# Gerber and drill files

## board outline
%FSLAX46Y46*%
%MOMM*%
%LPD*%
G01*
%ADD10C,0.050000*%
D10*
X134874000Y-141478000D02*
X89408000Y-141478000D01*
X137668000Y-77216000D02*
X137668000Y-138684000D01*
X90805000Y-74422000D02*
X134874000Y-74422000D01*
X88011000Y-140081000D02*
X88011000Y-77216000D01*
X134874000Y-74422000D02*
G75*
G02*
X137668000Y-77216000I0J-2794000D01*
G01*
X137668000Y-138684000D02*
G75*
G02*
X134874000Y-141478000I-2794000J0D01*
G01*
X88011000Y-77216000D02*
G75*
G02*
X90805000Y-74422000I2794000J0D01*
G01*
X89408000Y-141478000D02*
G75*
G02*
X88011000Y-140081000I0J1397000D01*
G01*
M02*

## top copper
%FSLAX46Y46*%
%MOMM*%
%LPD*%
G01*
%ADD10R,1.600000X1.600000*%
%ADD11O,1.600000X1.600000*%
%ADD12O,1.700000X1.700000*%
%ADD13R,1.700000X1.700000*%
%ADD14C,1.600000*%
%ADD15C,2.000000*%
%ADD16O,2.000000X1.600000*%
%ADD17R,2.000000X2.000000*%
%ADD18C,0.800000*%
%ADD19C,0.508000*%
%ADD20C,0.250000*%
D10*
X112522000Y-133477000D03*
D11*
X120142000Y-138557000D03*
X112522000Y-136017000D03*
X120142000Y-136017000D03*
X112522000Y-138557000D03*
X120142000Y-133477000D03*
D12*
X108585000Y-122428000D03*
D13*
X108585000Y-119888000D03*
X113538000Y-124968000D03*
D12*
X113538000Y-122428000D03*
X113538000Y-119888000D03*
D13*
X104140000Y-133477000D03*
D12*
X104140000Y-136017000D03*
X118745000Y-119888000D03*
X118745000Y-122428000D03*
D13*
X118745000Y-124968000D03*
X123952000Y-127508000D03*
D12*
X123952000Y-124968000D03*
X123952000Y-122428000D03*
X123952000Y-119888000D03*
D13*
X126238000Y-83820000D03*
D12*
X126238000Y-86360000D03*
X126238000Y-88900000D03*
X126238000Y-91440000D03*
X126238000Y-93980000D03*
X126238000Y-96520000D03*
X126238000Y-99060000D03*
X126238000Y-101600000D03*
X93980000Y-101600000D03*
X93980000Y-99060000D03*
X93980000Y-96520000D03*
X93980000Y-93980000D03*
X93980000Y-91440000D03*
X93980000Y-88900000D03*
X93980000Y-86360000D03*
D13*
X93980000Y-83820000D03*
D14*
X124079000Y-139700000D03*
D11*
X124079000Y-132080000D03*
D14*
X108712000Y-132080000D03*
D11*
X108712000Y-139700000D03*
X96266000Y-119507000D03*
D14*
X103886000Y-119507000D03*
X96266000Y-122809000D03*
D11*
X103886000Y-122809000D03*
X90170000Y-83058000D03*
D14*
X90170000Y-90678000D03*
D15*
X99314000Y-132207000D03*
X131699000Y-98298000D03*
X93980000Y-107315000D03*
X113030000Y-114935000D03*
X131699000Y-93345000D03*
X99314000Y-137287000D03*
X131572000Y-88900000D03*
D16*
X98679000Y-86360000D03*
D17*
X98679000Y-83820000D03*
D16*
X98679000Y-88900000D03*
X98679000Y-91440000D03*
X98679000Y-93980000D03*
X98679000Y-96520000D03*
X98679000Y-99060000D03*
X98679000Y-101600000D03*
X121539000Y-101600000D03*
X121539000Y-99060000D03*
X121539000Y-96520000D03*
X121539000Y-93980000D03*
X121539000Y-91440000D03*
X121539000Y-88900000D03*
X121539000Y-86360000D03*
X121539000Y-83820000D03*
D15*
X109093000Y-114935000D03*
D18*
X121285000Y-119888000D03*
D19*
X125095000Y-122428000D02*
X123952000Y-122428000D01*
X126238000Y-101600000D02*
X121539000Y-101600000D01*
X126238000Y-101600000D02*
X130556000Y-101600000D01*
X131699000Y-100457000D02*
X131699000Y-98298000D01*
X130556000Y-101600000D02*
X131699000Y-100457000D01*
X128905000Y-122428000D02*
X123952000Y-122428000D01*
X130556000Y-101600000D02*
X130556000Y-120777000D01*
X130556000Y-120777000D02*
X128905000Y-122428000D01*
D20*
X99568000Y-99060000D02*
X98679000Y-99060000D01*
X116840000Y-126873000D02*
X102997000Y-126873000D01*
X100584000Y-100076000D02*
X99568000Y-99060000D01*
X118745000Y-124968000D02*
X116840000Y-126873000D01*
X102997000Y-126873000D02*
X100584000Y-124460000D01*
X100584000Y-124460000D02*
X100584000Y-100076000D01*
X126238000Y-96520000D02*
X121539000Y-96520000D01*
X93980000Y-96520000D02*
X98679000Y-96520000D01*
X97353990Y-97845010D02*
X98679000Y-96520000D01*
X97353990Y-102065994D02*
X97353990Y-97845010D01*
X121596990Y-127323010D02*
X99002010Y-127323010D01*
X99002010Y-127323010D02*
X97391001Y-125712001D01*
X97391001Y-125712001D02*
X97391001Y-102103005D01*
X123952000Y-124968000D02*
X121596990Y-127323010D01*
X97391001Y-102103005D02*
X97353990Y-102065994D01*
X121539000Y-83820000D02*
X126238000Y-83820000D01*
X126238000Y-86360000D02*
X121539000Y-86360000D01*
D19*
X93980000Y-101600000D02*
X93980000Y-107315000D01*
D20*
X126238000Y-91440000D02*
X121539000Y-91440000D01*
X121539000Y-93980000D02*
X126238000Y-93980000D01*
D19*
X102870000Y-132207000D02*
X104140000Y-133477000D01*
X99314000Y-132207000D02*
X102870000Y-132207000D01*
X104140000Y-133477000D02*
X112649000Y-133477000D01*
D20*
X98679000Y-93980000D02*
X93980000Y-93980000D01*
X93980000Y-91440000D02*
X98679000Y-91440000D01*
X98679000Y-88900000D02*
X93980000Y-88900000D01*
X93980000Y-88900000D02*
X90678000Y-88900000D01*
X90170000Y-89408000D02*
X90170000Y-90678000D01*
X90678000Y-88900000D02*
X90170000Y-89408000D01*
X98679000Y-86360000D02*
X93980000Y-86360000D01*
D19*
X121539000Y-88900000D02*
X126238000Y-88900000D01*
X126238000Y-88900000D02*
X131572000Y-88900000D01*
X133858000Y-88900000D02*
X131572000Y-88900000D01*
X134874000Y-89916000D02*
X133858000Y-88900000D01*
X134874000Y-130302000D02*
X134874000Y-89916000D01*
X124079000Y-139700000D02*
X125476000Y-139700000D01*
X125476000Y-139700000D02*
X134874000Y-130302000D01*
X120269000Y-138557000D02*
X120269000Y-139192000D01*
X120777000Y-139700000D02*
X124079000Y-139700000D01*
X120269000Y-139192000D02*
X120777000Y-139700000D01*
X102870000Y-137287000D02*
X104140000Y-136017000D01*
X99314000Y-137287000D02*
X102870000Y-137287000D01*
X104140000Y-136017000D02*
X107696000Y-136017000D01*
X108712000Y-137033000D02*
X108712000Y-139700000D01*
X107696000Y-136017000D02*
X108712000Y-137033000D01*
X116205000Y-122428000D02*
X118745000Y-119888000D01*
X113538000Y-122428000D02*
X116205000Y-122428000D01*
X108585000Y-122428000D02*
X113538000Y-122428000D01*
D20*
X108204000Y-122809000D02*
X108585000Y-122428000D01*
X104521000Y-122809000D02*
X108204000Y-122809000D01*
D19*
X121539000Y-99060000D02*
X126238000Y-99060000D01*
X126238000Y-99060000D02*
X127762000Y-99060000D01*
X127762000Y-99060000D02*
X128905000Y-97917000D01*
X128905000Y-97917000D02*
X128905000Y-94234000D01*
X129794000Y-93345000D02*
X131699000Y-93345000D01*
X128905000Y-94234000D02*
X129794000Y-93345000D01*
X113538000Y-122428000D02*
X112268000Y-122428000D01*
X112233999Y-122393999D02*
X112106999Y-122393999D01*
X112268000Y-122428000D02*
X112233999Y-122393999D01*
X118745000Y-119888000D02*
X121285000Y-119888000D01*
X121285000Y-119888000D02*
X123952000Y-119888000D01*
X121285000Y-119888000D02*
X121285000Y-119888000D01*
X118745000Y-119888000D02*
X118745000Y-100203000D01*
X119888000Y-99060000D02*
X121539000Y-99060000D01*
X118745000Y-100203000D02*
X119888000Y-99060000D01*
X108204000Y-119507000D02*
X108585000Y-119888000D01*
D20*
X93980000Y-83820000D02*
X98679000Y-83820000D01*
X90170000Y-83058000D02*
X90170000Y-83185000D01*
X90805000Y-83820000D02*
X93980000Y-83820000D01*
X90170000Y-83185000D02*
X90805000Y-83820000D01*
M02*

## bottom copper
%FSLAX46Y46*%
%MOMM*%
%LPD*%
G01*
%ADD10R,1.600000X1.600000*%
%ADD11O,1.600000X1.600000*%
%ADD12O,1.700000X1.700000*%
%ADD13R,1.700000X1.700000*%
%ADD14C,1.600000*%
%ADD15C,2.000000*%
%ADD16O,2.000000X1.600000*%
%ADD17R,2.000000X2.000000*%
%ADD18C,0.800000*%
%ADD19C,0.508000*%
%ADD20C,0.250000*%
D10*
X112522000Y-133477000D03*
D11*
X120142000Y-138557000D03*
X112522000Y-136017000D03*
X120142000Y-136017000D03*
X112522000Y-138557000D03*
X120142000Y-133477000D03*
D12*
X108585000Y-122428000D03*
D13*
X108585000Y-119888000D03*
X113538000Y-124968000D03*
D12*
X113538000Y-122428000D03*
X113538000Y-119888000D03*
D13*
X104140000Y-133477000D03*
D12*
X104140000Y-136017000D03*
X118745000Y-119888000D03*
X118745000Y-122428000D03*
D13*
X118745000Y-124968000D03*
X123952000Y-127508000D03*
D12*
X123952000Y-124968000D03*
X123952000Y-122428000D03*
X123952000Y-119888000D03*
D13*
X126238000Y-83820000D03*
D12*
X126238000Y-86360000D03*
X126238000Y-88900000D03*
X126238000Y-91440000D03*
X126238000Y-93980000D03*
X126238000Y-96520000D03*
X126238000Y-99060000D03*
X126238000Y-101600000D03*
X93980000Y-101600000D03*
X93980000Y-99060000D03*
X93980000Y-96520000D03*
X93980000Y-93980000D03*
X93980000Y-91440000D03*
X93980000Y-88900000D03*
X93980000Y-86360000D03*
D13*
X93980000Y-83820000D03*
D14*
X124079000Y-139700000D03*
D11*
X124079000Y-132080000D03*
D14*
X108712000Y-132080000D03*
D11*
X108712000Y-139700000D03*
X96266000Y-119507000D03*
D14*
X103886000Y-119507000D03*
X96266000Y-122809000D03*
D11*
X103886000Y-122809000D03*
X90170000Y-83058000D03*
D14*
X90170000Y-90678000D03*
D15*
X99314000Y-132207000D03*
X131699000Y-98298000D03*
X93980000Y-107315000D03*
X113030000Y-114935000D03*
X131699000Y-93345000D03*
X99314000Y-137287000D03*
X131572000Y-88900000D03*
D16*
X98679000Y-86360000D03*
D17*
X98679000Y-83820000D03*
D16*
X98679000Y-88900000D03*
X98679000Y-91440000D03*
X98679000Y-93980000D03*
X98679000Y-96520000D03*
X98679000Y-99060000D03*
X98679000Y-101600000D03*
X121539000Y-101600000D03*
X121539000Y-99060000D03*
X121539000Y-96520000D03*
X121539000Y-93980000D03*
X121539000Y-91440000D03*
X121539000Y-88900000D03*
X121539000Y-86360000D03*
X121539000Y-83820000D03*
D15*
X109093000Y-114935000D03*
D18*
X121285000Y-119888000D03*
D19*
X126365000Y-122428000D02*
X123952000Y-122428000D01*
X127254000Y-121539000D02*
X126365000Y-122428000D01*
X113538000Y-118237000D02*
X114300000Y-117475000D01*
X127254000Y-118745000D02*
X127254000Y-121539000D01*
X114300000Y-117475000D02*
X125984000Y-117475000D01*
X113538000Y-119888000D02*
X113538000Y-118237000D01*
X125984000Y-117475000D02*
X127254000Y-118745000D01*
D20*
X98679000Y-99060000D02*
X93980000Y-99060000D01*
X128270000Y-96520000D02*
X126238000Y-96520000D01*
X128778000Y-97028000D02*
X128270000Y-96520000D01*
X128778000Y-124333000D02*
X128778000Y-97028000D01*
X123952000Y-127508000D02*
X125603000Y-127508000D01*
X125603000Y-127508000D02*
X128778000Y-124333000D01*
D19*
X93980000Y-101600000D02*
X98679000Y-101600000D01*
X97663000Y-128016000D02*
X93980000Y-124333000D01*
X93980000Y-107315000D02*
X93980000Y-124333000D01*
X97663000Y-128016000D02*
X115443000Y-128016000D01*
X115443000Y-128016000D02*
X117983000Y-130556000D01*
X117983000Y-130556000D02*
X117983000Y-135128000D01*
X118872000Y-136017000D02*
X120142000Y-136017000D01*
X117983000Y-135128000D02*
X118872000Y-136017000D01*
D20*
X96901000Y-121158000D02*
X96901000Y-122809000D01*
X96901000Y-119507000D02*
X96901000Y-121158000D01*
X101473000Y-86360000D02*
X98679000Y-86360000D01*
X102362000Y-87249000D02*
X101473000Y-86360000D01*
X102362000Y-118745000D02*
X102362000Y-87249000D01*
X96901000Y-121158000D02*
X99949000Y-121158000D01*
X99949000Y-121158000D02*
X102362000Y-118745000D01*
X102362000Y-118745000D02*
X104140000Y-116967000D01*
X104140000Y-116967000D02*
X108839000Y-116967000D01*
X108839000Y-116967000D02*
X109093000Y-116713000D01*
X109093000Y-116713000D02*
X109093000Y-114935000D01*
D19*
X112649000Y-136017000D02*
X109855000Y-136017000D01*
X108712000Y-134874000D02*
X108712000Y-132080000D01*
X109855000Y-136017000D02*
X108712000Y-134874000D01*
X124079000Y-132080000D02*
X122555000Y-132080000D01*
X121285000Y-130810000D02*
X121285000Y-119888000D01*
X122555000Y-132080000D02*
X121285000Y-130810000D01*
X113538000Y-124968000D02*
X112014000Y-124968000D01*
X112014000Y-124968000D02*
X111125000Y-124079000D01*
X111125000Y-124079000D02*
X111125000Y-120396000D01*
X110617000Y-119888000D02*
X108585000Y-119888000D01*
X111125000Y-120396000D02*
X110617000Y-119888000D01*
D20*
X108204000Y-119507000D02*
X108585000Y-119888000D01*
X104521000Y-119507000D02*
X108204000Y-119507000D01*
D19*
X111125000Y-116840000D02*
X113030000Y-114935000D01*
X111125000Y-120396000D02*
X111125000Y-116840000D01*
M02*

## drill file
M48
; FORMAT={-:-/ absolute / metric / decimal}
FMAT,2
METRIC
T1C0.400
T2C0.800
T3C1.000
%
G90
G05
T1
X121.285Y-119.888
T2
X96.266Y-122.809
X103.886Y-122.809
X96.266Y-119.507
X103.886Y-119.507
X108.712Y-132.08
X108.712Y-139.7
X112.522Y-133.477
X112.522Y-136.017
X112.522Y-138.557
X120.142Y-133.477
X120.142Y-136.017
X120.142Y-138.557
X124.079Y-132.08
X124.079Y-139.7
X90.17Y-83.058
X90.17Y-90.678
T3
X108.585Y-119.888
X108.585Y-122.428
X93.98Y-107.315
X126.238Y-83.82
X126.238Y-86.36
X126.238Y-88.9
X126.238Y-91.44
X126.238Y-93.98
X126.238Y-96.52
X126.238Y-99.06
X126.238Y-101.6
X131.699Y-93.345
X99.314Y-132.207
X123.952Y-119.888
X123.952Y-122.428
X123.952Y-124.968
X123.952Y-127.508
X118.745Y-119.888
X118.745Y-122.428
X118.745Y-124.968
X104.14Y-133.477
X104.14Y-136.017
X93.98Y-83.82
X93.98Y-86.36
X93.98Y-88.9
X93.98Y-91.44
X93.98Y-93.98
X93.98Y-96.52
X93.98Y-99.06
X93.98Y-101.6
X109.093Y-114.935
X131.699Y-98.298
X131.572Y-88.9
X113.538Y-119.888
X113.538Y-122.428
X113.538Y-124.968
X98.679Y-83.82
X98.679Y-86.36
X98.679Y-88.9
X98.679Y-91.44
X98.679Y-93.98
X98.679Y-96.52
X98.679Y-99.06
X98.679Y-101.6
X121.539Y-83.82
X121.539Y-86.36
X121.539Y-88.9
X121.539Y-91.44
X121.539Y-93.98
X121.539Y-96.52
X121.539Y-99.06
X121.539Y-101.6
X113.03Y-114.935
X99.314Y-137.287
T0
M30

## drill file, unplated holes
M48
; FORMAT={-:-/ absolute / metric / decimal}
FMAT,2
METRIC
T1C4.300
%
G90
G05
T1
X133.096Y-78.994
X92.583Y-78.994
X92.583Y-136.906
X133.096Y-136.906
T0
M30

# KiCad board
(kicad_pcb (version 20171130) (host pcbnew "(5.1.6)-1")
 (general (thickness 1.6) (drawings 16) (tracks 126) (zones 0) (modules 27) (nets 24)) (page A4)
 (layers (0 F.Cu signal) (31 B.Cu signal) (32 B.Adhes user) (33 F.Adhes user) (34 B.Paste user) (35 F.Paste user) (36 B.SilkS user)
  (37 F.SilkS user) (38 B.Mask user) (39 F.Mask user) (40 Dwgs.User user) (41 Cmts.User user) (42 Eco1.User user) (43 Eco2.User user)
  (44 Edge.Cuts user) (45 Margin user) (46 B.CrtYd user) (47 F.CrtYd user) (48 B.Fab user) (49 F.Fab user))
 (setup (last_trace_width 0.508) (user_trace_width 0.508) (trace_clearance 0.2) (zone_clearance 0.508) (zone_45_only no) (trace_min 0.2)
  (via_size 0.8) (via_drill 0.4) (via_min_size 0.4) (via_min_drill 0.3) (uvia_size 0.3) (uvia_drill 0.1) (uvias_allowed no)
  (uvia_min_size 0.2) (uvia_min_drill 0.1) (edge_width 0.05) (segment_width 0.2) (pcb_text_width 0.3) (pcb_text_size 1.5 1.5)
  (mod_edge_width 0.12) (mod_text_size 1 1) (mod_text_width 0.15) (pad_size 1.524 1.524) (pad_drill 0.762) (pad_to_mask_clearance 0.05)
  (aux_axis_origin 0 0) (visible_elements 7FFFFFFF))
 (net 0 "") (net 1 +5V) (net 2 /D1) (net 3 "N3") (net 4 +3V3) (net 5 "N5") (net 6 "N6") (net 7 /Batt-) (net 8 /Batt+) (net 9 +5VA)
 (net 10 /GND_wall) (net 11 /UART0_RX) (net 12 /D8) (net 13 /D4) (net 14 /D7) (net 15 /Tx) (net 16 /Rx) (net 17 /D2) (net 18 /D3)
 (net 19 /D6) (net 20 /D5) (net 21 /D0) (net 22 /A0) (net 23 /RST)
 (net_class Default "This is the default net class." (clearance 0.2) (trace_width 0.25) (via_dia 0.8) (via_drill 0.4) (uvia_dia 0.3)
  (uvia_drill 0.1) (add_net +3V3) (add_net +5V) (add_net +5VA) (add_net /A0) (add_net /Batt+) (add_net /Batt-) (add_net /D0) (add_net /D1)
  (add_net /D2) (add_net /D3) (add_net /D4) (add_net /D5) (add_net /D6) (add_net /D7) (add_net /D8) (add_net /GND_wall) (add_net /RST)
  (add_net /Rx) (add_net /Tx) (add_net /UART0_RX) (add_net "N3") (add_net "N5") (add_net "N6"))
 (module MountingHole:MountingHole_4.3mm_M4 (layer F.Cu) (at 92.583 136.906)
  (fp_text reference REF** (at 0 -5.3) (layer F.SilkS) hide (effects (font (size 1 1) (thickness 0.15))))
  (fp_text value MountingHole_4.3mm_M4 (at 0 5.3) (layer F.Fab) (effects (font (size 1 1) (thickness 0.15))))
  (pad 1 np_thru_hole circle (at 0 0) (size 4.3 4.3) (drill 4.3) (layers *.Cu *.Mask)))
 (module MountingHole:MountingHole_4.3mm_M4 (layer F.Cu) (at 133.096 136.906)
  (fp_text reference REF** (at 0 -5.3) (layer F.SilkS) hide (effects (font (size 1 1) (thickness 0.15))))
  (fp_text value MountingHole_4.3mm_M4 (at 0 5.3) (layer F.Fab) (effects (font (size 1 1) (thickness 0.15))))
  (pad 1 np_thru_hole circle (at 0 0) (size 4.3 4.3) (drill 4.3) (layers *.Cu *.Mask)))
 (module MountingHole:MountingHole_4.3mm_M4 (layer F.Cu) (at 92.583 78.994)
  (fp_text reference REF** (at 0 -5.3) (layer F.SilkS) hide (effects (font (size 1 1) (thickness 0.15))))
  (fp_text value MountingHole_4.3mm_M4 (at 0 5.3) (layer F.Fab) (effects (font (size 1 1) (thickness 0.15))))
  (pad 1 np_thru_hole circle (at 0 0) (size 4.3 4.3) (drill 4.3) (layers *.Cu *.Mask)))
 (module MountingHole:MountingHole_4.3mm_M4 (layer F.Cu) (at 133.096 78.994)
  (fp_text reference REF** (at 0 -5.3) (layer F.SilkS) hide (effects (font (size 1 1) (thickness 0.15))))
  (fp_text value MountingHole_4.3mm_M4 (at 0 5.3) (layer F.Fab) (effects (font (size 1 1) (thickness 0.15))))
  (pad 1 np_thru_hole circle (at 0 0) (size 4.3 4.3) (drill 4.3) (layers *.Cu *.Mask)))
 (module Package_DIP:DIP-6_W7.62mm (layer F.Cu) (at 112.522 133.477)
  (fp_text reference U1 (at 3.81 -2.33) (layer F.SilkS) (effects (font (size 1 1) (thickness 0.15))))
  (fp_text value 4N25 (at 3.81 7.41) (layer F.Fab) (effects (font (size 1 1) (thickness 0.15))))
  (pad 1 thru_hole rect (at 0 0) (size 1.6 1.6) (drill 0.8) (layers *.Cu *.Mask) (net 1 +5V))
  (pad 4 thru_hole oval (at 7.62 5.08) (size 1.6 1.6) (drill 0.8) (layers *.Cu *.Mask) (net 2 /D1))
  (pad 2 thru_hole oval (at 0 2.54) (size 1.6 1.6) (drill 0.8) (layers *.Cu *.Mask) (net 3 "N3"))
  (pad 5 thru_hole oval (at 7.62 2.54) (size 1.6 1.6) (drill 0.8) (layers *.Cu *.Mask) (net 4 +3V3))
  (pad 3 thru_hole oval (at 0 5.08) (size 1.6 1.6) (drill 0.8) (layers *.Cu *.Mask) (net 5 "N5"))
  (pad 6 thru_hole oval (at 7.62 0) (size 1.6 1.6) (drill 0.8) (layers *.Cu *.Mask) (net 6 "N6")))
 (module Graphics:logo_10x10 (layer B.Cu) (at 110.109 94.488 180)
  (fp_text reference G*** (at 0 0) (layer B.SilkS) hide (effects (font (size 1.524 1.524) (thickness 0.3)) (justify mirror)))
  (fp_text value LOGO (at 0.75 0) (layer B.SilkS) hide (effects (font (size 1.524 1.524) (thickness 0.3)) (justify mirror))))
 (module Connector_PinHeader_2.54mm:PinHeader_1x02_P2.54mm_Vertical (layer F.Cu) (at 108.585 119.888)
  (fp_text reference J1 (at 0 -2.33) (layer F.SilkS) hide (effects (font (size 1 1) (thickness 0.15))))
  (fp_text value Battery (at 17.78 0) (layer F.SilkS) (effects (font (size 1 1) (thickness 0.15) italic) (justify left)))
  (pad 2 thru_hole oval (at 0 2.54) (size 1.7 1.7) (drill 1) (layers *.Cu *.Mask) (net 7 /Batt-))
  (pad 1 thru_hole rect (at 0 0) (size 1.7 1.7) (drill 1) (layers *.Cu *.Mask) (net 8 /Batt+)))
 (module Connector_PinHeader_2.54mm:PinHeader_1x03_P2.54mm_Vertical (layer F.Cu) (at 113.538 124.968 180)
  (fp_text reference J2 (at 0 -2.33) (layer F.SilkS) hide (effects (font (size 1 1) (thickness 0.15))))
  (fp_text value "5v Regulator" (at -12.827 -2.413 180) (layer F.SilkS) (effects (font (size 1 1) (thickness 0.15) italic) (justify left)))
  (pad 1 thru_hole rect (at 0 0 180) (size 1.7 1.7) (drill 1) (layers *.Cu *.Mask) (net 8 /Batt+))
  (pad 2 thru_hole oval (at 0 2.54 180) (size 1.7 1.7) (drill 1) (layers *.Cu *.Mask) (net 7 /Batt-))
  (pad 3 thru_hole oval (at 0 5.08 180) (size 1.7 1.7) (drill 1) (layers *.Cu *.Mask) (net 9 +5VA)))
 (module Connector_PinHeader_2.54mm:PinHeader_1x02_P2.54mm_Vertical (layer F.Cu) (at 104.14 133.477)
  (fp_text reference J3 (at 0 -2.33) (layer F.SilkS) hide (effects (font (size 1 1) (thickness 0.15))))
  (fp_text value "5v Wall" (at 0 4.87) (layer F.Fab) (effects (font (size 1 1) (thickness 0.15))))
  (pad 1 thru_hole rect (at 0 0) (size 1.7 1.7) (drill 1) (layers *.Cu *.Mask) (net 1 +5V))
  (pad 2 thru_hole oval (at 0 2.54) (size 1.7 1.7) (drill 1) (layers *.Cu *.Mask) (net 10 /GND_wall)))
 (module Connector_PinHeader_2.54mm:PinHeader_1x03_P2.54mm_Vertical (layer F.Cu) (at 118.745 124.968 180)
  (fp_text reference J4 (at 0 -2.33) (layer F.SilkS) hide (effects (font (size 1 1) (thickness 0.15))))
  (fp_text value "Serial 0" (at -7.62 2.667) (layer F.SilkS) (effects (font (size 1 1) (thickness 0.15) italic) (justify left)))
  (pad 3 thru_hole oval (at 0 5.08 180) (size 1.7 1.7) (drill 1) (layers *.Cu *.Mask) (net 7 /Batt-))
  (pad 2 thru_hole oval (at 0 2.54 180) (size 1.7 1.7) (drill 1) (layers *.Cu *.Mask) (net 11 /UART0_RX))
  (pad 1 thru_hole rect (at 0 0 180) (size 1.7 1.7) (drill 1) (layers *.Cu *.Mask) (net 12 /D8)))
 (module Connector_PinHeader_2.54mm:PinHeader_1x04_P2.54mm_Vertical (layer F.Cu) (at 123.952 127.508 180)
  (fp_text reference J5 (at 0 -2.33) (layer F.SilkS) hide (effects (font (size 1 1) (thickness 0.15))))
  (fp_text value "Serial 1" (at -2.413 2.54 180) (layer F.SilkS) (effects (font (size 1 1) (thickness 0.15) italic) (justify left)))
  (pad 1 thru_hole rect (at 0 0 180) (size 1.7 1.7) (drill 1) (layers *.Cu *.Mask) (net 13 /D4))
  (pad 2 thru_hole oval (at 0 2.54 180) (size 1.7 1.7) (drill 1) (layers *.Cu *.Mask) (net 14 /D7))
  (pad 3 thru_hole oval (at 0 5.08 180) (size 1.7 1.7) (drill 1) (layers *.Cu *.Mask) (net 9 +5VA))
  (pad 4 thru_hole oval (at 0 7.62 180) (size 1.7 1.7) (drill 1) (layers *.Cu *.Mask) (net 7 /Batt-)))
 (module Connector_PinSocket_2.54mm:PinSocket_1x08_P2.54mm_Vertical (layer F.Cu) (at 126.238 83.82)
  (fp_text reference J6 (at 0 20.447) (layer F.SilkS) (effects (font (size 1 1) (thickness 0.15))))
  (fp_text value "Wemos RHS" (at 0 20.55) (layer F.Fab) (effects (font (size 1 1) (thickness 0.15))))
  (pad 1 thru_hole rect (at 0 0) (size 1.7 1.7) (drill 1) (layers *.Cu *.Mask) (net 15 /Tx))
  (pad 2 thru_hole oval (at 0 2.54) (size 1.7 1.7) (drill 1) (layers *.Cu *.Mask) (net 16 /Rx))
  (pad 3 thru_hole oval (at 0 5.08) (size 1.7 1.7) (drill 1) (layers *.Cu *.Mask) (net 2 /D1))
  (pad 4 thru_hole oval (at 0 7.62) (size 1.7 1.7) (drill 1) (layers *.Cu *.Mask) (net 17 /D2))
  (pad 5 thru_hole oval (at 0 10.16) (size 1.7 1.7) (drill 1) (layers *.Cu *.Mask) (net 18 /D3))
  (pad 6 thru_hole oval (at 0 12.7) (size 1.7 1.7) (drill 1) (layers *.Cu *.Mask) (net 13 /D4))
  (pad 7 thru_hole oval (at 0 15.24) (size 1.7 1.7) (drill 1) (layers *.Cu *.Mask) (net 7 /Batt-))
  (pad 8 thru_hole oval (at 0 17.78) (size 1.7 1.7) (drill 1) (layers *.Cu *.Mask) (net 9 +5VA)))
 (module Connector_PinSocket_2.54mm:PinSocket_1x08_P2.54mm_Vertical (layer F.Cu) (at 93.98 83.82)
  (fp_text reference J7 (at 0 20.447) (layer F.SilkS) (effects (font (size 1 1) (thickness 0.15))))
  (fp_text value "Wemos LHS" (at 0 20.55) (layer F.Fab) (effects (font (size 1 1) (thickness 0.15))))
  (pad 8 thru_hole oval (at 0 17.78) (size 1.7 1.7) (drill 1) (layers *.Cu *.Mask) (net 4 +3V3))
  (pad 7 thru_hole oval (at 0 15.24) (size 1.7 1.7) (drill 1) (layers *.Cu *.Mask) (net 12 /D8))
  (pad 6 thru_hole oval (at 0 12.7) (size 1.7 1.7) (drill 1) (layers *.Cu *.Mask) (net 14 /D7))
  (pad 5 thru_hole oval (at 0 10.16) (size 1.7 1.7) (drill 1) (layers *.Cu *.Mask) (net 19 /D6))
  (pad 4 thru_hole oval (at 0 7.62) (size 1.7 1.7) (drill 1) (layers *.Cu *.Mask) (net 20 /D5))
  (pad 3 thru_hole oval (at 0 5.08) (size 1.7 1.7) (drill 1) (layers *.Cu *.Mask) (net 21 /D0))
  (pad 2 thru_hole oval (at 0 2.54) (size 1.7 1.7) (drill 1) (layers *.Cu *.Mask) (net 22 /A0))
  (pad 1 thru_hole rect (at 0 0) (size 1.7 1.7) (drill 1) (layers *.Cu *.Mask) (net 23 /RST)))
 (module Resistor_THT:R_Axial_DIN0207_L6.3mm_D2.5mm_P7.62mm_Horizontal (layer F.Cu) (at 124.079 139.7 90)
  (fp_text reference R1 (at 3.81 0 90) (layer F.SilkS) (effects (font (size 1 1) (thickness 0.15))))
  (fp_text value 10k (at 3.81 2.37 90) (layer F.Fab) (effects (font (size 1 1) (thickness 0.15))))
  (pad 1 thru_hole circle (at 0 0 90) (size 1.6 1.6) (drill 0.8) (layers *.Cu *.Mask) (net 2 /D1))
  (pad 2 thru_hole oval (at 7.62 0 90) (size 1.6 1.6) (drill 0.8) (layers *.Cu *.Mask) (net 7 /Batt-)))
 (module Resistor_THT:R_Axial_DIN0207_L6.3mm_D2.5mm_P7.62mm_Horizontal (layer F.Cu) (at 108.712 132.08 270)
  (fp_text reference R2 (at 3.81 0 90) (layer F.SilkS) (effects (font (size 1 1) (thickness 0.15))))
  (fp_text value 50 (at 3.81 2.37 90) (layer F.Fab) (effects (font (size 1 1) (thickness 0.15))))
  (pad 1 thru_hole circle (at 0 0 270) (size 1.6 1.6) (drill 0.8) (layers *.Cu *.Mask) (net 3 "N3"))
  (pad 2 thru_hole oval (at 7.62 0 270) (size 1.6 1.6) (drill 0.8) (layers *.Cu *.Mask) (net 10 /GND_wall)))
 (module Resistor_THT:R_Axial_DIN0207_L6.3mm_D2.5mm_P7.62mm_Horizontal (layer F.Cu) (at 103.886 119.507 180)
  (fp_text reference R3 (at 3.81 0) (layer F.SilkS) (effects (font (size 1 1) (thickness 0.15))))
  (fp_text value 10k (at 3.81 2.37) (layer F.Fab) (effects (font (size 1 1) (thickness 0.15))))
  (pad 2 thru_hole oval (at 7.62 0 180) (size 1.6 1.6) (drill 0.8) (layers *.Cu *.Mask) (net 22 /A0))
  (pad 1 thru_hole circle (at 0 0 180) (size 1.6 1.6) (drill 0.8) (layers *.Cu *.Mask) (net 8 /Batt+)))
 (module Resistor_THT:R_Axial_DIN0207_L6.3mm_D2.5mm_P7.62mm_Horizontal (layer F.Cu) (at 96.266 122.809)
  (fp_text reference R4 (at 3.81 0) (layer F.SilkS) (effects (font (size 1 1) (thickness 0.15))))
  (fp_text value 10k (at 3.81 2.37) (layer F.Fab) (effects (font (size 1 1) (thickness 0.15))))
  (pad 1 thru_hole circle (at 0 0) (size 1.6 1.6) (drill 0.8) (layers *.Cu *.Mask) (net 22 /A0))
  (pad 2 thru_hole oval (at 7.62 0) (size 1.6 1.6) (drill 0.8) (layers *.Cu *.Mask) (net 7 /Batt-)))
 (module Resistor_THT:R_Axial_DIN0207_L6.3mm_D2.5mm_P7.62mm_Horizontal (layer F.Cu) (at 90.17 90.678 90)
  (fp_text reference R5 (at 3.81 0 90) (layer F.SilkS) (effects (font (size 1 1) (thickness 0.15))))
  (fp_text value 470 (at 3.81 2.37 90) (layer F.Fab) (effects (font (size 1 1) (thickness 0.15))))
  (pad 2 thru_hole oval (at 7.62 0 90) (size 1.6 1.6) (drill 0.8) (layers *.Cu *.Mask) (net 23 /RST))
  (pad 1 thru_hole circle (at 0 0 90) (size 1.6 1.6) (drill 0.8) (layers *.Cu *.Mask) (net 21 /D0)))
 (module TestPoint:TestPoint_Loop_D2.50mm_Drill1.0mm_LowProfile (layer F.Cu) (at 99.314 132.207)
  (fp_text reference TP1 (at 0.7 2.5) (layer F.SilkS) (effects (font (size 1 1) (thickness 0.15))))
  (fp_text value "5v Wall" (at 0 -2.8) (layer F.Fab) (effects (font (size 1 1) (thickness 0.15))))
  (pad 1 thru_hole circle (at 0 0) (size 2 2) (drill 1) (layers *.Cu *.Mask) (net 1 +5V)))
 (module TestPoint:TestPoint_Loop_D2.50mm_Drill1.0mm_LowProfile (layer F.Cu) (at 131.699 98.298)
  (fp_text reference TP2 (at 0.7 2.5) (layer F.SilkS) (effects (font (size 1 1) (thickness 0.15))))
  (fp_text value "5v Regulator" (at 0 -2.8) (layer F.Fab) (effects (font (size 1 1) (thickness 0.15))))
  (pad 1 thru_hole circle (at 0 0) (size 2 2) (drill 1) (layers *.Cu *.Mask) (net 9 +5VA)))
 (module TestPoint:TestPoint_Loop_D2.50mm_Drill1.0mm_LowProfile (layer F.Cu) (at 93.98 107.315)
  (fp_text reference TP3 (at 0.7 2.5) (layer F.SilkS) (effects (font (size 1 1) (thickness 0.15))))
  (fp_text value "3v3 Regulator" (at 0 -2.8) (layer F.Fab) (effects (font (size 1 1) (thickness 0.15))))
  (pad 1 thru_hole circle (at 0 0) (size 2 2) (drill 1) (layers *.Cu *.Mask) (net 4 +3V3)))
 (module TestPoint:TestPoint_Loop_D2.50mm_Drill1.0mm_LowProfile (layer F.Cu) (at 113.03 114.935)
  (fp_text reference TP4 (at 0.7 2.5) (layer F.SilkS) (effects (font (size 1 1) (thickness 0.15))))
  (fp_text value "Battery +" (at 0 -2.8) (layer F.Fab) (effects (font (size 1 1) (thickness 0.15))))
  (pad 1 thru_hole circle (at 0 0) (size 2 2) (drill 1) (layers *.Cu *.Mask) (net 8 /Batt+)))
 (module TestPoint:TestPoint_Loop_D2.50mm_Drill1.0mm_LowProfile (layer F.Cu) (at 131.699 93.345)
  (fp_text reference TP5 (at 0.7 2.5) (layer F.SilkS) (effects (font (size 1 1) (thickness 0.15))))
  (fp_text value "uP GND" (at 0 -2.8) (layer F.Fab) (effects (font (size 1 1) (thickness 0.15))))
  (pad 1 thru_hole circle (at 0 0) (size 2 2) (drill 1) (layers *.Cu *.Mask) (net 7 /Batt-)))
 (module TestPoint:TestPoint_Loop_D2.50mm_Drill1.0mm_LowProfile (layer F.Cu) (at 99.314 137.287)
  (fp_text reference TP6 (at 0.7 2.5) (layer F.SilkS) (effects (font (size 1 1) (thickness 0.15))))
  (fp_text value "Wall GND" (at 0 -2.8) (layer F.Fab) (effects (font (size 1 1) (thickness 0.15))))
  (pad 1 thru_hole circle (at 0 0) (size 2 2) (drill 1) (layers *.Cu *.Mask) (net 10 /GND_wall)))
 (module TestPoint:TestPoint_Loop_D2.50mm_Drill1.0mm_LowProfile (layer F.Cu) (at 131.572 88.9)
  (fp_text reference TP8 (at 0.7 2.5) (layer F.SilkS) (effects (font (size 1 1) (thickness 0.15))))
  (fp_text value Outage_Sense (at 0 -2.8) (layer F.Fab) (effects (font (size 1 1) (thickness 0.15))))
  (pad 1 thru_hole circle (at 0 0) (size 2 2) (drill 1) (layers *.Cu *.Mask) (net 2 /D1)))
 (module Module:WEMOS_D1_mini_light (layer F.Cu) (at 98.679 83.82)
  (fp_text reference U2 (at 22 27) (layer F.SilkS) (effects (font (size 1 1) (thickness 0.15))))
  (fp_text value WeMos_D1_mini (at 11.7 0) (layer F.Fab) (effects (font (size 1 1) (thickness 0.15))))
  (pad 2 thru_hole oval (at 0 2.54) (size 2 1.6) (drill 1) (layers *.Cu *.Mask) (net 22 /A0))
  (pad 1 thru_hole rect (at 0 0) (size 2 2) (drill 1) (layers *.Cu *.Mask) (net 23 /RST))
  (pad 3 thru_hole oval (at 0 5.08) (size 2 1.6) (drill 1) (layers *.Cu *.Mask) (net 21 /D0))
  (pad 4 thru_hole oval (at 0 7.62) (size 2 1.6) (drill 1) (layers *.Cu *.Mask) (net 20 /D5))
  (pad 5 thru_hole oval (at 0 10.16) (size 2 1.6) (drill 1) (layers *.Cu *.Mask) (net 19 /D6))
  (pad 6 thru_hole oval (at 0 12.7) (size 2 1.6) (drill 1) (layers *.Cu *.Mask) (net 14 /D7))
  (pad 7 thru_hole oval (at 0 15.24) (size 2 1.6) (drill 1) (layers *.Cu *.Mask) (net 12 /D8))
  (pad 8 thru_hole oval (at 0 17.78) (size 2 1.6) (drill 1) (layers *.Cu *.Mask) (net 4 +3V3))
  (pad 9 thru_hole oval (at 22.86 17.78) (size 2 1.6) (drill 1) (layers *.Cu *.Mask) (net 9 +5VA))
  (pad 10 thru_hole oval (at 22.86 15.24) (size 2 1.6) (drill 1) (layers *.Cu *.Mask) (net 7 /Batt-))
  (pad 11 thru_hole oval (at 22.86 12.7) (size 2 1.6) (drill 1) (layers *.Cu *.Mask) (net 13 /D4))
  (pad 12 thru_hole oval (at 22.86 10.16) (size 2 1.6) (drill 1) (layers *.Cu *.Mask) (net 18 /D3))
  (pad 13 thru_hole oval (at 22.86 7.62) (size 2 1.6) (drill 1) (layers *.Cu *.Mask) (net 17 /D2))
  (pad 14 thru_hole oval (at 22.86 5.08) (size 2 1.6) (drill 1) (layers *.Cu *.Mask) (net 2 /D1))
  (pad 15 thru_hole oval (at 22.86 2.54) (size 2 1.6) (drill 1) (layers *.Cu *.Mask) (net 16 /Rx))
  (pad 16 thru_hole oval (at 22.86 0) (size 2 1.6) (drill 1) (layers *.Cu *.Mask) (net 15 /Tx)))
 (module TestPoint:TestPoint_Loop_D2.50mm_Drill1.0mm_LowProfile (layer F.Cu) (at 109.093 114.935)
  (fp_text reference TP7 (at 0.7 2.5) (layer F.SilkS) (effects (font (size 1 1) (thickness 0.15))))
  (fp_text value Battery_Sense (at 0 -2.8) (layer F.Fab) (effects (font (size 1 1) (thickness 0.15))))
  (pad 1 thru_hole circle (at 0 0) (size 2 2) (drill 1) (layers *.Cu *.Mask) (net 22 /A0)))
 (gr_line (start 134.874 141.478) (end 89.408 141.478) (layer Edge.Cuts) (width 0.05))
 (gr_line (start 137.668 77.216) (end 137.668 138.684) (layer Edge.Cuts) (width 0.05))
 (gr_line (start 90.805 74.422) (end 134.874 74.422) (layer Edge.Cuts) (width 0.05))
 (gr_line (start 88.011 140.081) (end 88.011 77.216) (layer Edge.Cuts) (width 0.05))
 (gr_arc (start 134.874 77.216) (end 137.668 77.216) (angle -90) (layer Edge.Cuts) (width 0.05))
 (gr_arc (start 134.874 138.684) (end 134.874 141.478) (angle -90) (layer Edge.Cuts) (width 0.05))
 (gr_arc (start 90.805 77.216) (end 90.805 74.422) (angle -90) (layer Edge.Cuts) (width 0.05))
 (gr_arc (start 89.408 140.081) (end 88.011 140.081) (angle -90) (layer Edge.Cuts) (width 0.05))
 (segment (start 125.095 122.428) (end 123.952 122.428) (width 0.508) (layer F.Cu) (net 9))
 (segment (start 126.238 101.6) (end 121.539 101.6) (width 0.508) (layer F.Cu) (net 9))
 (segment (start 126.238 101.6) (end 130.556 101.6) (width 0.508) (layer F.Cu) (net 9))
 (segment (start 131.699 100.457) (end 131.699 98.298) (width 0.508) (layer F.Cu) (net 9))
 (segment (start 130.556 101.6) (end 131.699 100.457) (width 0.508) (layer F.Cu) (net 9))
 (segment (start 126.365 122.428) (end 123.952 122.428) (width 0.508) (layer B.Cu) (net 9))
 (segment (start 127.254 121.539) (end 126.365 122.428) (width 0.508) (layer B.Cu) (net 9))
 (segment (start 113.538 118.237) (end 114.3 117.475) (width 0.508) (layer B.Cu) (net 9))
 (segment (start 127.254 118.745) (end 127.254 121.539) (width 0.508) (layer B.Cu) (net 9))
 (segment (start 114.3 117.475) (end 125.984 117.475) (width 0.508) (layer B.Cu) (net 9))
 (segment (start 113.538 119.888) (end 113.538 118.237) (width 0.508) (layer B.Cu) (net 9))
 (segment (start 125.984 117.475) (end 127.254 118.745) (width 0.508) (layer B.Cu) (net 9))
 (segment (start 128.905 122.428) (end 123.952 122.428) (width 0.508) (layer F.Cu) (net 9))
 (segment (start 130.556 101.6) (end 130.556 120.777) (width 0.508) (layer F.Cu) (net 9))
 (segment (start 130.556 120.777) (end 128.905 122.428) (width 0.508) (layer F.Cu) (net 9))
 (segment (start 98.679 99.06) (end 93.98 99.06) (width 0.25) (layer B.Cu) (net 12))
 (segment (start 99.568 99.06) (end 98.679 99.06) (width 0.25) (layer F.Cu) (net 12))
 (segment (start 116.84 126.873) (end 102.997 126.873) (width 0.25) (layer F.Cu) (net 12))
 (segment (start 100.584 100.076) (end 99.568 99.06) (width 0.25) (layer F.Cu) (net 12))
 (segment (start 118.745 124.968) (end 116.84 126.873) (width 0.25) (layer F.Cu) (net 12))
 (segment (start 102.997 126.873) (end 100.584 124.46) (width 0.25) (layer F.Cu) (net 12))
 (segment (start 100.584 124.46) (end 100.584 100.076) (width 0.25) (layer F.Cu) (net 12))
 (segment (start 126.238 96.52) (end 121.539 96.52) (width 0.25) (layer F.Cu) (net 13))
 (segment (start 128.27 96.52) (end 126.238 96.52) (width 0.25) (layer B.Cu) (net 13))
 (segment (start 128.778 97.028) (end 128.27 96.52) (width 0.25) (layer B.Cu) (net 13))
 (segment (start 128.778 124.333) (end 128.778 97.028) (width 0.25) (layer B.Cu) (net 13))
 (segment (start 123.952 127.508) (end 125.603 127.508) (width 0.25) (layer B.Cu) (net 13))
 (segment (start 125.603 127.508) (end 128.778 124.333) (width 0.25) (layer B.Cu) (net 13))
 (segment (start 93.98 96.52) (end 98.679 96.52) (width 0.25) (layer F.Cu) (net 14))
 (segment (start 97.35399 97.84501) (end 98.679 96.52) (width 0.25) (layer F.Cu) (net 14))
 (segment (start 97.35399 102.065994) (end 97.35399 97.84501) (width 0.25) (layer F.Cu) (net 14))
 (segment (start 121.59699 127.32301) (end 99.00201 127.32301) (width 0.25) (layer F.Cu) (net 14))
 (segment (start 99.00201 127.32301) (end 97.391001 125.712001) (width 0.25) (layer F.Cu) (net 14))
 (segment (start 97.391001 125.712001) (end 97.391001 102.103005) (width 0.25) (layer F.Cu) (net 14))
 (segment (start 123.952 124.968) (end 121.59699 127.32301) (width 0.25) (layer F.Cu) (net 14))
 (segment (start 97.391001 102.103005) (end 97.35399 102.065994) (width 0.25) (layer F.Cu) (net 14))
 (segment (start 121.539 83.82) (end 126.238 83.82) (width 0.25) (layer F.Cu) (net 15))
 (segment (start 126.238 86.36) (end 121.539 86.36) (width 0.25) (layer F.Cu) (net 16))
 (segment (start 93.98 101.6) (end 98.679 101.6) (width 0.508) (layer B.Cu) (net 4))
 (segment (start 93.98 101.6) (end 93.98 107.315) (width 0.508) (layer F.Cu) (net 4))
 (segment (start 97.663 128.016) (end 93.98 124.333) (width 0.508) (layer B.Cu) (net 4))
 (segment (start 93.98 107.315) (end 93.98 124.333) (width 0.508) (layer B.Cu) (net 4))
 (segment (start 97.663 128.016) (end 115.443 128.016) (width 0.508) (layer B.Cu) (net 4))
 (segment (start 115.443 128.016) (end 117.983 130.556) (width 0.508) (layer B.Cu) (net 4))
 (segment (start 117.983 130.556) (end 117.983 135.128) (width 0.508) (layer B.Cu) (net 4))
 (segment (start 118.872 136.017) (end 120.142 136.017) (width 0.508) (layer B.Cu) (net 4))
 (segment (start 117.983 135.128) (end 118.872 136.017) (width 0.508) (layer B.Cu) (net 4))
 (segment (start 126.238 91.44) (end 121.539 91.44) (width 0.25) (layer F.Cu) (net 17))
 (segment (start 121.539 93.98) (end 126.238 93.98) (width 0.25) (layer F.Cu) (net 18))
 (segment (start 102.87 132.207) (end 104.14 133.477) (width 0.508) (layer F.Cu) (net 1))
 (segment (start 99.314 132.207) (end 102.87 132.207) (width 0.508) (layer F.Cu) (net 1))
 (segment (start 104.14 133.477) (end 112.649 133.477) (width 0.508) (layer F.Cu) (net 1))
 (segment (start 98.679 93.98) (end 93.98 93.98) (width 0.25) (layer F.Cu) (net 19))
 (segment (start 93.98 91.44) (end 98.679 91.44) (width 0.25) (layer F.Cu) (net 20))
 (segment (start 98.679 88.9) (end 93.98 88.9) (width 0.25) (layer F.Cu) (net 21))
 (segment (start 93.98 88.9) (end 90.678 88.9) (width 0.25) (layer F.Cu) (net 21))
 (segment (start 90.17 89.408) (end 90.17 90.678) (width 0.25) (layer F.Cu) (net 21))
 (segment (start 90.678 88.9) (end 90.17 89.408) (width 0.25) (layer F.Cu) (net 21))
 (segment (start 98.679 86.36) (end 93.98 86.36) (width 0.25) (layer F.Cu) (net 22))
 (segment (start 96.901 121.158) (end 96.901 122.809) (width 0.25) (layer B.Cu) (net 22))
 (segment (start 96.901 119.507) (end 96.901 121.158) (width 0.25) (layer B.Cu) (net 22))
 (segment (start 101.473 86.36) (end 98.679 86.36) (width 0.25) (layer B.Cu) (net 22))
 (segment (start 102.362 87.249) (end 101.473 86.36) (width 0.25) (layer B.Cu) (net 22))
 (segment (start 102.362 118.745) (end 102.362 87.249) (width 0.25) (layer B.Cu) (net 22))
 (segment (start 96.901 121.158) (end 99.949 121.158) (width 0.25) (layer B.Cu) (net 22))
 (segment (start 99.949 121.158) (end 102.362 118.745) (width 0.25) (layer B.Cu) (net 22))
 (segment (start 102.362 118.745) (end 104.14 116.967) (width 0.25) (layer B.Cu) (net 22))
 (segment (start 104.14 116.967) (end 108.839 116.967) (width 0.25) (layer B.Cu) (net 22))
 (segment (start 108.839 116.967) (end 109.093 116.713) (width 0.25) (layer B.Cu) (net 22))
 (segment (start 109.093 116.713) (end 109.093 114.935) (width 0.25) (layer B.Cu) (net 22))
 (segment (start 112.649 136.017) (end 109.855 136.017) (width 0.508) (layer B.Cu) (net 3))
 (segment (start 108.712 134.874) (end 108.712 132.08) (width 0.508) (layer B.Cu) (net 3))
 (segment (start 109.855 136.017) (end 108.712 134.874) (width 0.508) (layer B.Cu) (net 3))
 (segment (start 121.539 88.9) (end 126.238 88.9) (width 0.508) (layer F.Cu) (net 2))
 (segment (start 126.238 88.9) (end 131.572 88.9) (width 0.508) (layer F.Cu) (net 2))
 (segment (start 133.858 88.9) (end 131.572 88.9) (width 0.508) (layer F.Cu) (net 2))
 (segment (start 134.874 89.916) (end 133.858 88.9) (width 0.508) (layer F.Cu) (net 2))
 (segment (start 134.874 130.302) (end 134.874 89.916) (width 0.508) (layer F.Cu) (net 2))
 (segment (start 124.079 139.7) (end 125.476 139.7) (width 0.508) (layer F.Cu) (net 2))
 (segment (start 125.476 139.7) (end 134.874 130.302) (width 0.508) (layer F.Cu) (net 2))
 (segment (start 120.269 138.557) (end 120.269 139.192) (width 0.508) (layer F.Cu) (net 2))
 (segment (start 120.777 139.7) (end 124.079 139.7) (width 0.508) (layer F.Cu) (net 2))
 (segment (start 120.269 139.192) (end 120.777 139.7) (width 0.508) (layer F.Cu) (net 2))
 (segment (start 102.87 137.287) (end 104.14 136.017) (width 0.508) (layer F.Cu) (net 10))
 (segment (start 99.314 137.287) (end 102.87 137.287) (width 0.508) (layer F.Cu) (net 10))
 (segment (start 104.14 136.017) (end 107.696 136.017) (width 0.508) (layer F.Cu) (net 10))
 (segment (start 108.712 137.033) (end 108.712 139.7) (width 0.508) (layer F.Cu) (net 10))
 (segment (start 107.696 136.017) (end 108.712 137.033) (width 0.508) (layer F.Cu) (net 10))
 (segment (start 116.205 122.428) (end 118.745 119.888) (width 0.508) (layer F.Cu) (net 7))
 (segment (start 113.538 122.428) (end 116.205 122.428) (width 0.508) (layer F.Cu) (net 7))
 (segment (start 108.585 122.428) (end 113.538 122.428) (width 0.508) (layer F.Cu) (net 7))
 (segment (start 108.204 122.809) (end 108.585 122.428) (width 0.25) (layer F.Cu) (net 7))
 (segment (start 104.521 122.809) (end 108.204 122.809) (width 0.25) (layer F.Cu) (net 7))
 (segment (start 121.539 99.06) (end 126.238 99.06) (width 0.508) (layer F.Cu) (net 7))
 (segment (start 126.238 99.06) (end 127.762 99.06) (width 0.508) (layer F.Cu) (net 7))
 (segment (start 127.762 99.06) (end 128.905 97.917) (width 0.508) (layer F.Cu) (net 7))
 (segment (start 128.905 97.917) (end 128.905 94.234) (width 0.508) (layer F.Cu) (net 7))
 (segment (start 129.794 93.345) (end 131.699 93.345) (width 0.508) (layer F.Cu) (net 7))
 (segment (start 128.905 94.234) (end 129.794 93.345) (width 0.508) (layer F.Cu) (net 7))
 (segment (start 113.538 122.428) (end 112.268 122.428) (width 0.508) (layer F.Cu) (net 7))
 (segment (start 112.233999 122.393999) (end 112.106999 122.393999) (width 0.508) (layer F.Cu) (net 7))
 (segment (start 112.268 122.428) (end 112.233999 122.393999) (width 0.508) (layer F.Cu) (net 7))
 (segment (start 124.079 132.08) (end 122.555 132.08) (width 0.508) (layer B.Cu) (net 7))
 (segment (start 121.285 130.81) (end 121.285 119.888) (width 0.508) (layer B.Cu) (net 7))
 (segment (start 122.555 132.08) (end 121.285 130.81) (width 0.508) (layer B.Cu) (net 7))
 (segment (start 118.745 119.888) (end 121.285 119.888) (width 0.508) (layer F.Cu) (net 7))
 (segment (start 121.285 119.888) (end 123.952 119.888) (width 0.508) (layer F.Cu) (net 7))
 (segment (start 121.285 119.888) (end 121.285 119.888) (width 0.508) (layer F.Cu) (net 7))
 (via (at 121.285 119.888) (size 0.8) (drill 0.4) (layers F.Cu B.Cu) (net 7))
 (segment (start 118.745 119.888) (end 118.745 100.203) (width 0.508) (layer F.Cu) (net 7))
 (segment (start 119.888 99.06) (end 121.539 99.06) (width 0.508) (layer F.Cu) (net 7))
 (segment (start 118.745 100.203) (end 119.888 99.06) (width 0.508) (layer F.Cu) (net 7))
 (segment (start 113.538 124.968) (end 112.014 124.968) (width 0.508) (layer B.Cu) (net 8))
 (segment (start 112.014 124.968) (end 111.125 124.079) (width 0.508) (layer B.Cu) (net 8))
 (segment (start 111.125 124.079) (end 111.125 120.396) (width 0.508) (layer B.Cu) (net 8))
 (segment (start 110.617 119.888) (end 108.585 119.888) (width 0.508) (layer B.Cu) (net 8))
 (segment (start 111.125 120.396) (end 110.617 119.888) (width 0.508) (layer B.Cu) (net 8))
 (segment (start 108.204 119.507) (end 108.585 119.888) (width 0.25) (layer B.Cu) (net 8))
 (segment (start 104.521 119.507) (end 108.204 119.507) (width 0.25) (layer B.Cu) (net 8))
 (segment (start 108.204 119.507) (end 108.585 119.888) (width 0.508) (layer F.Cu) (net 8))
 (segment (start 111.125 116.84) (end 113.03 114.935) (width 0.508) (layer B.Cu) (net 8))
 (segment (start 111.125 120.396) (end 111.125 116.84) (width 0.508) (layer B.Cu) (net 8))
 (segment (start 93.98 83.82) (end 98.679 83.82) (width 0.25) (layer F.Cu) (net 23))
 (segment (start 90.17 83.058) (end 90.17 83.185) (width 0.25) (layer F.Cu) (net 23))
 (segment (start 90.805 83.82) (end 93.98 83.82) (width 0.25) (layer F.Cu) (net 23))
 (segment (start 90.17 83.185) (end 90.805 83.82) (width 0.25) (layer F.Cu) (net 23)))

